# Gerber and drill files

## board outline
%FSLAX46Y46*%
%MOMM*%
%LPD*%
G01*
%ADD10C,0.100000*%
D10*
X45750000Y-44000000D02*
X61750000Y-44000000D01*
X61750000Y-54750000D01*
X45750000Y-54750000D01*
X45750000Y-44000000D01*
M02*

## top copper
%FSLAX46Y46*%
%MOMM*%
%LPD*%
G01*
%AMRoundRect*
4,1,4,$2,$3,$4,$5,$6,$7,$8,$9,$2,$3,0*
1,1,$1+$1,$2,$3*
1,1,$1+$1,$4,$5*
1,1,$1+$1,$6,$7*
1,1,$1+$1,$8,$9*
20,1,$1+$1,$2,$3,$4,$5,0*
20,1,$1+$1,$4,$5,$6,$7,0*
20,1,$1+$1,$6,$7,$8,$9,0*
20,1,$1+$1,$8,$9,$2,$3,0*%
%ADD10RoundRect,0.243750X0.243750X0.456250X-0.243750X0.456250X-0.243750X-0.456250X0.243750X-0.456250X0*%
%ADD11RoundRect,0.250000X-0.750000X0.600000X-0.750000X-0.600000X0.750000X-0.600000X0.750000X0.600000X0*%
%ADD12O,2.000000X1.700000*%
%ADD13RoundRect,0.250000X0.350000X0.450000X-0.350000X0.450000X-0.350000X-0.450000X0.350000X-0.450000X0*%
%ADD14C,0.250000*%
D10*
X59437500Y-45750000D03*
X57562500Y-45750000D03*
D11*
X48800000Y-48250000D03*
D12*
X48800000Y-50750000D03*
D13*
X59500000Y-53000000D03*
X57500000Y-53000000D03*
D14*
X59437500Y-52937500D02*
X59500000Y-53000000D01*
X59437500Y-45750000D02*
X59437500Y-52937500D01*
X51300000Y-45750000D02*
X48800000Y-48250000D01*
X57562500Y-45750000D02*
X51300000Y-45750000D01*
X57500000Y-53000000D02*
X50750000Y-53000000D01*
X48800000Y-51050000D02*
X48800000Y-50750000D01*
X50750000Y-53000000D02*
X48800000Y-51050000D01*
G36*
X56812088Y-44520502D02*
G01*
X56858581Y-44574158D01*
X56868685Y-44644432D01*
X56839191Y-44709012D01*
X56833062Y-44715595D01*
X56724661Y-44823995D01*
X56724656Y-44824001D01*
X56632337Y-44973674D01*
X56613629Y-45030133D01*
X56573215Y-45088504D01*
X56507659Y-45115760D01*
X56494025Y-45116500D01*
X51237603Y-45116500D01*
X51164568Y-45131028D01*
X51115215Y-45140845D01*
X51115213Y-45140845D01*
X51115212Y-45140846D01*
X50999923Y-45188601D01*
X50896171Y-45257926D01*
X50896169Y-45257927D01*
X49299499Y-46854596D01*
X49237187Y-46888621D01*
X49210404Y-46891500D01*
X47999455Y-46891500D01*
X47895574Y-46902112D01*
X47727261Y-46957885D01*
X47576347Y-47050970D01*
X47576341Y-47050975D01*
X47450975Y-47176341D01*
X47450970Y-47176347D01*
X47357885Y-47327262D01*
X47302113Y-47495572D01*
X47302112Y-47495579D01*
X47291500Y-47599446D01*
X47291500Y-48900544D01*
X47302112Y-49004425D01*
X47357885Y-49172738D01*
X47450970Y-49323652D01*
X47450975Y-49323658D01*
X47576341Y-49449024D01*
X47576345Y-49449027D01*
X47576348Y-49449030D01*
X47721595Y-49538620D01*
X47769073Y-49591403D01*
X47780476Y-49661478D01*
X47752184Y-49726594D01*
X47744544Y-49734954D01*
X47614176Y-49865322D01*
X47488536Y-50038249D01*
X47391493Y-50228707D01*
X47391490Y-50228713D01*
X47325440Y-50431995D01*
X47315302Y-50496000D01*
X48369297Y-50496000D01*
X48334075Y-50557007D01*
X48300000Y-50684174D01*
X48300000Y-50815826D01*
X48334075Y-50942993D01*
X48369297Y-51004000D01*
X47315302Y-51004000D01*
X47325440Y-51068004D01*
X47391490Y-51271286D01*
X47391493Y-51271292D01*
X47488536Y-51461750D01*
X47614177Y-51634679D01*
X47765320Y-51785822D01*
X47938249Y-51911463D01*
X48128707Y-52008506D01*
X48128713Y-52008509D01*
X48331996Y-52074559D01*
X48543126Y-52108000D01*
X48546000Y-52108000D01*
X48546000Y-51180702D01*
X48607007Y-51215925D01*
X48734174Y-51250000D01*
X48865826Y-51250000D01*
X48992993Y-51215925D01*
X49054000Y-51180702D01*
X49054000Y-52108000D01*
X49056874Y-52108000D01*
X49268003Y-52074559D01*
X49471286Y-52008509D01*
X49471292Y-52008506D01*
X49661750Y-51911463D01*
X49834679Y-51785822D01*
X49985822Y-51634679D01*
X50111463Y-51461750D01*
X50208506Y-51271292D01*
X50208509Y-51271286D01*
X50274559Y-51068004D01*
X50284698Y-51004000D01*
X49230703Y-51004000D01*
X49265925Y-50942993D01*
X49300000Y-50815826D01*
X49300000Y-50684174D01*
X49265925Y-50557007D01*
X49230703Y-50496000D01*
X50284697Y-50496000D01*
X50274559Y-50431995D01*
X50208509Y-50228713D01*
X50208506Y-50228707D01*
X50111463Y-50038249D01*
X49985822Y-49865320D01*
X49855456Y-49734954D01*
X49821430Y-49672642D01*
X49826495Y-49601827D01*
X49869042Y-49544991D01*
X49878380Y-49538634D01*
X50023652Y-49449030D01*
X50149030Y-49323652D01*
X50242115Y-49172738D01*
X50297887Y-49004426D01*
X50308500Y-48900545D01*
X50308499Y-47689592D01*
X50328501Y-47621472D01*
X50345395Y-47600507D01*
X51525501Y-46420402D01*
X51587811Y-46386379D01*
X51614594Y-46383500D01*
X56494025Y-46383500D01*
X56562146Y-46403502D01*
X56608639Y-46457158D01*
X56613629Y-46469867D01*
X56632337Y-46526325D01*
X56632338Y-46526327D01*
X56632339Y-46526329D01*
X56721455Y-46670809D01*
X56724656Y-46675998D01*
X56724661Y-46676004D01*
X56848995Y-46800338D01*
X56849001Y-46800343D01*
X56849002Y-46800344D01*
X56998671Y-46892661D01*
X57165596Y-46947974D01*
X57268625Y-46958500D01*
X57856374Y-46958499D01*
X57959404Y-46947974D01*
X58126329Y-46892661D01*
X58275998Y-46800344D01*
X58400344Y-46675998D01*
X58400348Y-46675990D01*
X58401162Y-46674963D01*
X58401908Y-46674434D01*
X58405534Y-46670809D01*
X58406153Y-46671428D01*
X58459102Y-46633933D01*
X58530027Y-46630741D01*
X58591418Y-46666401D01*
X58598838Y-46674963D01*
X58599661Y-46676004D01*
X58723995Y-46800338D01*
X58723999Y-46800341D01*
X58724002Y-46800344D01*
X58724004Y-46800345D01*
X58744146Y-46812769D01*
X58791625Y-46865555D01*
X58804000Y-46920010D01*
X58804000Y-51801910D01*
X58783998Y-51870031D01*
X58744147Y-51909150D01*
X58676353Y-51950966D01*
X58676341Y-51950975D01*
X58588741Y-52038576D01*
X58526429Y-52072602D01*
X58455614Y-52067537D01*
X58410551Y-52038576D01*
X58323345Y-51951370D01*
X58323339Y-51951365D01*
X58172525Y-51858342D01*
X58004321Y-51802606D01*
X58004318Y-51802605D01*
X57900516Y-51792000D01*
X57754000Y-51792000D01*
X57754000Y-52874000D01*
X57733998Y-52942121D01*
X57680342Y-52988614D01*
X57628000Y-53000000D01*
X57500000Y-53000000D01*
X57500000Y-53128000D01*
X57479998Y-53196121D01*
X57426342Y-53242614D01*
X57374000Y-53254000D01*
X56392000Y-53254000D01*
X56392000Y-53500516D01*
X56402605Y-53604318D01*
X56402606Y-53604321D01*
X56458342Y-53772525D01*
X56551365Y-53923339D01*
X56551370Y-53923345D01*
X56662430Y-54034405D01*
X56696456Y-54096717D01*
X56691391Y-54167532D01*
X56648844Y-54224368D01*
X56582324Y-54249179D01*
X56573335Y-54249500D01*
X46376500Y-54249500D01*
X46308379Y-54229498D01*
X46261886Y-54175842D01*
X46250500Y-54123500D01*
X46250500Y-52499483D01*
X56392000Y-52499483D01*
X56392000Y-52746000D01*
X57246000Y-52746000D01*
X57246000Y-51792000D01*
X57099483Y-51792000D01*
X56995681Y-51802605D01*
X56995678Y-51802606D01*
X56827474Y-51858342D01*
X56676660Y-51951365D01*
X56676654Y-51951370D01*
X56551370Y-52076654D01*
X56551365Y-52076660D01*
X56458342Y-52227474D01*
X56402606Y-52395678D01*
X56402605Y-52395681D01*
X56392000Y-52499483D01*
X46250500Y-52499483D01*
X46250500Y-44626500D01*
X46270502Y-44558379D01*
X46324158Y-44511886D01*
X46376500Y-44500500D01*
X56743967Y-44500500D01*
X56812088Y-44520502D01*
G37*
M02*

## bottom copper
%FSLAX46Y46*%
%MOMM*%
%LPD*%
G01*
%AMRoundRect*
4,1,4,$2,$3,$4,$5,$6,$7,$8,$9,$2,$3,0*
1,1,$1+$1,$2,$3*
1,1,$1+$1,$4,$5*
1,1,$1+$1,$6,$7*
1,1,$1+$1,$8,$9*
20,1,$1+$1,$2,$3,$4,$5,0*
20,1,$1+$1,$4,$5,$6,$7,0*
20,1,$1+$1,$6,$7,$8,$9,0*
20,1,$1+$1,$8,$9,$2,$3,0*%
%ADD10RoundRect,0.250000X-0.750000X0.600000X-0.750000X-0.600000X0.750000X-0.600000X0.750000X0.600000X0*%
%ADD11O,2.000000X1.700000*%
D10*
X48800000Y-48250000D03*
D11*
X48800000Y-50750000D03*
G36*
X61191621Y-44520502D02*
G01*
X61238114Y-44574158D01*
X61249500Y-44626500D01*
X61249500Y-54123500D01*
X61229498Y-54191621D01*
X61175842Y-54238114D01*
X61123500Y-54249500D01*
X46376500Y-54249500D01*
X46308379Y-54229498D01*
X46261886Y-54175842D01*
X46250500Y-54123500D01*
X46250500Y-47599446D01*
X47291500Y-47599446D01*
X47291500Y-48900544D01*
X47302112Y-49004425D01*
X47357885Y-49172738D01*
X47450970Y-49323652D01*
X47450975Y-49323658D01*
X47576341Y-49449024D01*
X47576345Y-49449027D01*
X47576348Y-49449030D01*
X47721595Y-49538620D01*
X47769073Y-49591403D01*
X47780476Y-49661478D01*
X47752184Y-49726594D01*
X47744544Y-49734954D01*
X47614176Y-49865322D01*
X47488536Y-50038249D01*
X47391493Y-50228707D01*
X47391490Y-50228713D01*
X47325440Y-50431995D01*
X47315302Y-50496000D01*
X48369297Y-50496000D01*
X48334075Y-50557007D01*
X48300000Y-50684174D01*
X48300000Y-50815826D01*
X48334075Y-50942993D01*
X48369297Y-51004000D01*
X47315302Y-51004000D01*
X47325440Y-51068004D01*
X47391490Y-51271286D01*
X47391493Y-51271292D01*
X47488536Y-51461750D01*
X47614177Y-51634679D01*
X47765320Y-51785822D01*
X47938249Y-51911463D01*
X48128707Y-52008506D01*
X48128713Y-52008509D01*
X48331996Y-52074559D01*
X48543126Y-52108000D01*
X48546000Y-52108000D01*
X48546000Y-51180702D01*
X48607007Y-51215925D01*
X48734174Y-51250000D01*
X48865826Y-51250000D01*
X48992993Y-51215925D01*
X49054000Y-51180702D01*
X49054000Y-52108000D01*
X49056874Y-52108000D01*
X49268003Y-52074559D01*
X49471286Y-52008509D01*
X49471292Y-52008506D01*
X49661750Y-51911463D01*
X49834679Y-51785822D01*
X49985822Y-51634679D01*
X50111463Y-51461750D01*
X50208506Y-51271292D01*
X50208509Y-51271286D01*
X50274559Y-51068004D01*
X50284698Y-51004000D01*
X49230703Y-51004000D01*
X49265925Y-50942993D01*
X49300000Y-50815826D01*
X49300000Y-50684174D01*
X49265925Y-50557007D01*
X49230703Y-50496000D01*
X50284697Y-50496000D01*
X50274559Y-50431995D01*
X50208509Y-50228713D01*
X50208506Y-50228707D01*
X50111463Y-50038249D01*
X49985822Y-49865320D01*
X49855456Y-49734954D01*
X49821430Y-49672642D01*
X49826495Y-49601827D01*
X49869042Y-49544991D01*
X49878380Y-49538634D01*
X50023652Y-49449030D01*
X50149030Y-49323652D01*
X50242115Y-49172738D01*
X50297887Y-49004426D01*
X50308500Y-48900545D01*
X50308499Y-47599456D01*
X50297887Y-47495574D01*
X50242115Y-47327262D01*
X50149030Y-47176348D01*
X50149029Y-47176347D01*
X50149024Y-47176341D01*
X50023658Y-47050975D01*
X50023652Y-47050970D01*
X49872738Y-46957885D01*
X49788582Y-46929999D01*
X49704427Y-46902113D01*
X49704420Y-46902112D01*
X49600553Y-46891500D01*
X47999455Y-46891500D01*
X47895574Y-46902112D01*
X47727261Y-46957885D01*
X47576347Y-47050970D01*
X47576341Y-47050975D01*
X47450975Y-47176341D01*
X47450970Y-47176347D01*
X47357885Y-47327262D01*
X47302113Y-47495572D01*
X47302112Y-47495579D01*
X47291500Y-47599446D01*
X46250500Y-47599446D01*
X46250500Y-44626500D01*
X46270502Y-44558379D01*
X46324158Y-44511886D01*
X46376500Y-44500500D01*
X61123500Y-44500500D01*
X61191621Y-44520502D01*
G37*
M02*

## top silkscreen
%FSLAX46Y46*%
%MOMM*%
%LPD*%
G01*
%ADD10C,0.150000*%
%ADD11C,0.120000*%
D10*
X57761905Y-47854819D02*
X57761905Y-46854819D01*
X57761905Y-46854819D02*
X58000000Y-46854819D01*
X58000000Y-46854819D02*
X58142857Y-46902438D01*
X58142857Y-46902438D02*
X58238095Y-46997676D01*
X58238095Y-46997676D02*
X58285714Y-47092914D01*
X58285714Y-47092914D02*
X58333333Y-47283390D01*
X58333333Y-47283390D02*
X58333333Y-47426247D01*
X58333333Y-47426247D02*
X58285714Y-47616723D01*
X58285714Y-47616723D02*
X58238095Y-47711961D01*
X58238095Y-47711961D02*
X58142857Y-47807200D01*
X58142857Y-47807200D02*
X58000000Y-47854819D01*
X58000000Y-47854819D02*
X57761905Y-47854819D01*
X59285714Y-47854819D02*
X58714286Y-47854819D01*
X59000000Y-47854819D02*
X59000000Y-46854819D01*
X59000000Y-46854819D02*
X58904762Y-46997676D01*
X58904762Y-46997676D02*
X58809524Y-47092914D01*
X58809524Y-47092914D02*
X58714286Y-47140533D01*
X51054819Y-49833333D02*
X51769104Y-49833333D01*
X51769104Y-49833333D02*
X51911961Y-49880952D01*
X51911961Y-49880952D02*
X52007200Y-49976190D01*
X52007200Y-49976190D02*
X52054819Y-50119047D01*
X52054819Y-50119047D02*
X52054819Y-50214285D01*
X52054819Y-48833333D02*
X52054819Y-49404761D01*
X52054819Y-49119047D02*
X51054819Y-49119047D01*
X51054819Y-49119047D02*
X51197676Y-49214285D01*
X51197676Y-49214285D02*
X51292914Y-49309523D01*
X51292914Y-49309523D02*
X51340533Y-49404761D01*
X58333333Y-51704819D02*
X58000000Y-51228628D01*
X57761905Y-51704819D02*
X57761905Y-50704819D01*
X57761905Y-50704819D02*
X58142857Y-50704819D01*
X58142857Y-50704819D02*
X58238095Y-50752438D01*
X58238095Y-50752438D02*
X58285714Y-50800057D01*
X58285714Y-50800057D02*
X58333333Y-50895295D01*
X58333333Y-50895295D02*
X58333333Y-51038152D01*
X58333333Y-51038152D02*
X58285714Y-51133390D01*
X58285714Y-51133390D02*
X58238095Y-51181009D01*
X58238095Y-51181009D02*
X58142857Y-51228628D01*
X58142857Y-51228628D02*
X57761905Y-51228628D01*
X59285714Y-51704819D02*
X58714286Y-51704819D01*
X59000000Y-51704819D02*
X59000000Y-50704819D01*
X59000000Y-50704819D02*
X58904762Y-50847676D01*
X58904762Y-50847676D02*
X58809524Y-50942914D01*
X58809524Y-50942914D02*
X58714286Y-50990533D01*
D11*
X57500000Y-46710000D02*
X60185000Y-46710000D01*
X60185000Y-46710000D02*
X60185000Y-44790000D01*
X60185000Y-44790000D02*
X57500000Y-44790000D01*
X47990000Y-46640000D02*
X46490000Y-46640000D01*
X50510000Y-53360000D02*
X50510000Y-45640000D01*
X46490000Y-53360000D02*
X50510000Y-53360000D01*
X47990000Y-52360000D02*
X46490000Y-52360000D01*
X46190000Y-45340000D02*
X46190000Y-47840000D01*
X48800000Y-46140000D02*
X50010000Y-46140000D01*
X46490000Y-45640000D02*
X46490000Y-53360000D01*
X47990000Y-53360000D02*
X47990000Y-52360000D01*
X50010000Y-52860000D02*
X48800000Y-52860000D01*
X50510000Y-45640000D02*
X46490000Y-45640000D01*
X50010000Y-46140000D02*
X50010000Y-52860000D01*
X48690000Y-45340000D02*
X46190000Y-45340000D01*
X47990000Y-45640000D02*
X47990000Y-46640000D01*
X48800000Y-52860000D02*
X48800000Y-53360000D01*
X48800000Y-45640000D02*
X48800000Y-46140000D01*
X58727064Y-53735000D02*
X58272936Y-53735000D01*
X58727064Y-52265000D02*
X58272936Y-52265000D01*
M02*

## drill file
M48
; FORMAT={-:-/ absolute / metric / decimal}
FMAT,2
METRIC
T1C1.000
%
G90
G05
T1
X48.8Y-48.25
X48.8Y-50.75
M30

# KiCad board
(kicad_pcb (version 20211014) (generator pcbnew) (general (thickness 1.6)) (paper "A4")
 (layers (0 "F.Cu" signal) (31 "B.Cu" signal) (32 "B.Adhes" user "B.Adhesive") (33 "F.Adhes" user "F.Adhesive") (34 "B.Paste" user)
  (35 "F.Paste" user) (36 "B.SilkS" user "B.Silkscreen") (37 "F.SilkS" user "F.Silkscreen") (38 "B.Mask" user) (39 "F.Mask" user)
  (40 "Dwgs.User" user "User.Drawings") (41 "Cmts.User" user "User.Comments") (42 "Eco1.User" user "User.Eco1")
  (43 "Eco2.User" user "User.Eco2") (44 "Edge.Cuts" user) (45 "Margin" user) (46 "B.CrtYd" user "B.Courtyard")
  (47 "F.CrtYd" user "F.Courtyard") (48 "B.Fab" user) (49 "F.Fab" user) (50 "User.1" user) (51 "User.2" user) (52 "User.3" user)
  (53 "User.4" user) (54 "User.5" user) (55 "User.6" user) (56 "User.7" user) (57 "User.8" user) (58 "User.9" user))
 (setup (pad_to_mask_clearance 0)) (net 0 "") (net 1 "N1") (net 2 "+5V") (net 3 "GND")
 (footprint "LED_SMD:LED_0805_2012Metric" (layer "F.Cu") (at 58.5 45.75 180)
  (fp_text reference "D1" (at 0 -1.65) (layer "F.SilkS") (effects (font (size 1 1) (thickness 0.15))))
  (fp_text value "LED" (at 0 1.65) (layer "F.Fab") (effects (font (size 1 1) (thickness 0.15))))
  (fp_line (start 1 -0.96) (end -1.685 -0.96) (layer "F.SilkS") (width 0.12))
  (fp_line (start -1.685 -0.96) (end -1.685 0.96) (layer "F.SilkS") (width 0.12))
  (fp_line (start -1.685 0.96) (end 1 0.96) (layer "F.SilkS") (width 0.12))
  (pad "1" smd roundrect (at -0.9375 0 180) (size 0.975 1.4) (layers "F.Cu" "F.Paste" "F.Mask") (roundrect_rratio 0.25) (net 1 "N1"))
  (pad "2" smd roundrect (at 0.9375 0 180) (size 0.975 1.4) (layers "F.Cu" "F.Paste" "F.Mask") (roundrect_rratio 0.25) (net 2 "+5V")))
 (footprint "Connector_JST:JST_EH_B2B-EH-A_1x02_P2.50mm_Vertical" (layer "F.Cu") (at 48.8 48.25 -90)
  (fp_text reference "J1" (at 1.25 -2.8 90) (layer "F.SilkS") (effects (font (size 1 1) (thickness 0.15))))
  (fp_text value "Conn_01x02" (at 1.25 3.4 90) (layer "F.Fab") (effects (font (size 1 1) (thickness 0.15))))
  (fp_line (start -1.61 0.81) (end -1.61 2.31) (layer "F.SilkS") (width 0.12))
  (fp_line (start 5.11 -1.71) (end -2.61 -1.71) (layer "F.SilkS") (width 0.12))
  (fp_line (start 5.11 2.31) (end 5.11 -1.71) (layer "F.SilkS") (width 0.12))
  (fp_line (start 4.11 0.81) (end 4.11 2.31) (layer "F.SilkS") (width 0.12))
  (fp_line (start -2.91 2.61) (end -0.41 2.61) (layer "F.SilkS") (width 0.12))
  (fp_line (start -2.11 0) (end -2.11 -1.21) (layer "F.SilkS") (width 0.12))
  (fp_line (start -2.61 2.31) (end 5.11 2.31) (layer "F.SilkS") (width 0.12))
  (fp_line (start 5.11 0.81) (end 4.11 0.81) (layer "F.SilkS") (width 0.12))
  (fp_line (start 4.61 -1.21) (end 4.61 0) (layer "F.SilkS") (width 0.12))
  (fp_line (start -2.61 -1.71) (end -2.61 2.31) (layer "F.SilkS") (width 0.12))
  (fp_line (start -2.11 -1.21) (end 4.61 -1.21) (layer "F.SilkS") (width 0.12))
  (fp_line (start -2.91 0.11) (end -2.91 2.61) (layer "F.SilkS") (width 0.12))
  (fp_line (start -2.61 0.81) (end -1.61 0.81) (layer "F.SilkS") (width 0.12))
  (fp_line (start 4.61 0) (end 5.11 0) (layer "F.SilkS") (width 0.12))
  (fp_line (start -2.61 0) (end -2.11 0) (layer "F.SilkS") (width 0.12))
  (pad "1" thru_hole roundrect (at 0 0 270) (size 1.7 2) (drill 1) (layers *.Cu *.Mask) (roundrect_rratio 0.1470588235) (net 2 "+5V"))
  (pad "2" thru_hole oval (at 2.5 0 270) (size 1.7 2) (drill 1) (layers *.Cu *.Mask) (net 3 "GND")))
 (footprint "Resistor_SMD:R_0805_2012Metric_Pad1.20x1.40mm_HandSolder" (layer "F.Cu") (at 58.5 53 180)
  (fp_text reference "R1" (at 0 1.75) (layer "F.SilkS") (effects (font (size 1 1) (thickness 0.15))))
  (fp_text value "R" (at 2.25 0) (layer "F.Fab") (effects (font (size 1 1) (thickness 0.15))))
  (fp_line (start -0.227064 -0.735) (end 0.227064 -0.735) (layer "F.SilkS") (width 0.12))
  (fp_line (start -0.227064 0.735) (end 0.227064 0.735) (layer "F.SilkS") (width 0.12))
  (pad "1" smd roundrect (at -1 0 180) (size 1.2 1.4) (layers "F.Cu" "F.Paste" "F.Mask") (roundrect_rratio 0.2083333333) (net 1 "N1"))
  (pad "2" smd roundrect (at 1 0 180) (size 1.2 1.4) (layers "F.Cu" "F.Paste" "F.Mask") (roundrect_rratio 0.2083333333) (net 3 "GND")))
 (gr_rect (start 61.75 54.75) (end 45.75 44) (layer "Edge.Cuts") (width 0.1) (fill none))
 (segment (start 59.4375 52.9375) (end 59.5 53) (width 0.25) (layer "F.Cu") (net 1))
 (segment (start 59.4375 45.75) (end 59.4375 52.9375) (width 0.25) (layer "F.Cu") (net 1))
 (segment (start 51.3 45.75) (end 48.8 48.25) (width 0.25) (layer "F.Cu") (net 2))
 (segment (start 57.5625 45.75) (end 51.3 45.75) (width 0.25) (layer "F.Cu") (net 2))
 (segment (start 57.5 53) (end 50.75 53) (width 0.25) (layer "F.Cu") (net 3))
 (segment (start 48.8 51.05) (end 48.8 50.75) (width 0.25) (layer "F.Cu") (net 3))
 (segment (start 50.75 53) (end 48.8 51.05) (width 0.25) (layer "F.Cu") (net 3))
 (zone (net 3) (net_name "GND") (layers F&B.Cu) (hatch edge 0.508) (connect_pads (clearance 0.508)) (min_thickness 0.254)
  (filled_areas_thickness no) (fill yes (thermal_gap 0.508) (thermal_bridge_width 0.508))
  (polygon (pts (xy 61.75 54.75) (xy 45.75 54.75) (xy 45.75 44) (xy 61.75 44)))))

